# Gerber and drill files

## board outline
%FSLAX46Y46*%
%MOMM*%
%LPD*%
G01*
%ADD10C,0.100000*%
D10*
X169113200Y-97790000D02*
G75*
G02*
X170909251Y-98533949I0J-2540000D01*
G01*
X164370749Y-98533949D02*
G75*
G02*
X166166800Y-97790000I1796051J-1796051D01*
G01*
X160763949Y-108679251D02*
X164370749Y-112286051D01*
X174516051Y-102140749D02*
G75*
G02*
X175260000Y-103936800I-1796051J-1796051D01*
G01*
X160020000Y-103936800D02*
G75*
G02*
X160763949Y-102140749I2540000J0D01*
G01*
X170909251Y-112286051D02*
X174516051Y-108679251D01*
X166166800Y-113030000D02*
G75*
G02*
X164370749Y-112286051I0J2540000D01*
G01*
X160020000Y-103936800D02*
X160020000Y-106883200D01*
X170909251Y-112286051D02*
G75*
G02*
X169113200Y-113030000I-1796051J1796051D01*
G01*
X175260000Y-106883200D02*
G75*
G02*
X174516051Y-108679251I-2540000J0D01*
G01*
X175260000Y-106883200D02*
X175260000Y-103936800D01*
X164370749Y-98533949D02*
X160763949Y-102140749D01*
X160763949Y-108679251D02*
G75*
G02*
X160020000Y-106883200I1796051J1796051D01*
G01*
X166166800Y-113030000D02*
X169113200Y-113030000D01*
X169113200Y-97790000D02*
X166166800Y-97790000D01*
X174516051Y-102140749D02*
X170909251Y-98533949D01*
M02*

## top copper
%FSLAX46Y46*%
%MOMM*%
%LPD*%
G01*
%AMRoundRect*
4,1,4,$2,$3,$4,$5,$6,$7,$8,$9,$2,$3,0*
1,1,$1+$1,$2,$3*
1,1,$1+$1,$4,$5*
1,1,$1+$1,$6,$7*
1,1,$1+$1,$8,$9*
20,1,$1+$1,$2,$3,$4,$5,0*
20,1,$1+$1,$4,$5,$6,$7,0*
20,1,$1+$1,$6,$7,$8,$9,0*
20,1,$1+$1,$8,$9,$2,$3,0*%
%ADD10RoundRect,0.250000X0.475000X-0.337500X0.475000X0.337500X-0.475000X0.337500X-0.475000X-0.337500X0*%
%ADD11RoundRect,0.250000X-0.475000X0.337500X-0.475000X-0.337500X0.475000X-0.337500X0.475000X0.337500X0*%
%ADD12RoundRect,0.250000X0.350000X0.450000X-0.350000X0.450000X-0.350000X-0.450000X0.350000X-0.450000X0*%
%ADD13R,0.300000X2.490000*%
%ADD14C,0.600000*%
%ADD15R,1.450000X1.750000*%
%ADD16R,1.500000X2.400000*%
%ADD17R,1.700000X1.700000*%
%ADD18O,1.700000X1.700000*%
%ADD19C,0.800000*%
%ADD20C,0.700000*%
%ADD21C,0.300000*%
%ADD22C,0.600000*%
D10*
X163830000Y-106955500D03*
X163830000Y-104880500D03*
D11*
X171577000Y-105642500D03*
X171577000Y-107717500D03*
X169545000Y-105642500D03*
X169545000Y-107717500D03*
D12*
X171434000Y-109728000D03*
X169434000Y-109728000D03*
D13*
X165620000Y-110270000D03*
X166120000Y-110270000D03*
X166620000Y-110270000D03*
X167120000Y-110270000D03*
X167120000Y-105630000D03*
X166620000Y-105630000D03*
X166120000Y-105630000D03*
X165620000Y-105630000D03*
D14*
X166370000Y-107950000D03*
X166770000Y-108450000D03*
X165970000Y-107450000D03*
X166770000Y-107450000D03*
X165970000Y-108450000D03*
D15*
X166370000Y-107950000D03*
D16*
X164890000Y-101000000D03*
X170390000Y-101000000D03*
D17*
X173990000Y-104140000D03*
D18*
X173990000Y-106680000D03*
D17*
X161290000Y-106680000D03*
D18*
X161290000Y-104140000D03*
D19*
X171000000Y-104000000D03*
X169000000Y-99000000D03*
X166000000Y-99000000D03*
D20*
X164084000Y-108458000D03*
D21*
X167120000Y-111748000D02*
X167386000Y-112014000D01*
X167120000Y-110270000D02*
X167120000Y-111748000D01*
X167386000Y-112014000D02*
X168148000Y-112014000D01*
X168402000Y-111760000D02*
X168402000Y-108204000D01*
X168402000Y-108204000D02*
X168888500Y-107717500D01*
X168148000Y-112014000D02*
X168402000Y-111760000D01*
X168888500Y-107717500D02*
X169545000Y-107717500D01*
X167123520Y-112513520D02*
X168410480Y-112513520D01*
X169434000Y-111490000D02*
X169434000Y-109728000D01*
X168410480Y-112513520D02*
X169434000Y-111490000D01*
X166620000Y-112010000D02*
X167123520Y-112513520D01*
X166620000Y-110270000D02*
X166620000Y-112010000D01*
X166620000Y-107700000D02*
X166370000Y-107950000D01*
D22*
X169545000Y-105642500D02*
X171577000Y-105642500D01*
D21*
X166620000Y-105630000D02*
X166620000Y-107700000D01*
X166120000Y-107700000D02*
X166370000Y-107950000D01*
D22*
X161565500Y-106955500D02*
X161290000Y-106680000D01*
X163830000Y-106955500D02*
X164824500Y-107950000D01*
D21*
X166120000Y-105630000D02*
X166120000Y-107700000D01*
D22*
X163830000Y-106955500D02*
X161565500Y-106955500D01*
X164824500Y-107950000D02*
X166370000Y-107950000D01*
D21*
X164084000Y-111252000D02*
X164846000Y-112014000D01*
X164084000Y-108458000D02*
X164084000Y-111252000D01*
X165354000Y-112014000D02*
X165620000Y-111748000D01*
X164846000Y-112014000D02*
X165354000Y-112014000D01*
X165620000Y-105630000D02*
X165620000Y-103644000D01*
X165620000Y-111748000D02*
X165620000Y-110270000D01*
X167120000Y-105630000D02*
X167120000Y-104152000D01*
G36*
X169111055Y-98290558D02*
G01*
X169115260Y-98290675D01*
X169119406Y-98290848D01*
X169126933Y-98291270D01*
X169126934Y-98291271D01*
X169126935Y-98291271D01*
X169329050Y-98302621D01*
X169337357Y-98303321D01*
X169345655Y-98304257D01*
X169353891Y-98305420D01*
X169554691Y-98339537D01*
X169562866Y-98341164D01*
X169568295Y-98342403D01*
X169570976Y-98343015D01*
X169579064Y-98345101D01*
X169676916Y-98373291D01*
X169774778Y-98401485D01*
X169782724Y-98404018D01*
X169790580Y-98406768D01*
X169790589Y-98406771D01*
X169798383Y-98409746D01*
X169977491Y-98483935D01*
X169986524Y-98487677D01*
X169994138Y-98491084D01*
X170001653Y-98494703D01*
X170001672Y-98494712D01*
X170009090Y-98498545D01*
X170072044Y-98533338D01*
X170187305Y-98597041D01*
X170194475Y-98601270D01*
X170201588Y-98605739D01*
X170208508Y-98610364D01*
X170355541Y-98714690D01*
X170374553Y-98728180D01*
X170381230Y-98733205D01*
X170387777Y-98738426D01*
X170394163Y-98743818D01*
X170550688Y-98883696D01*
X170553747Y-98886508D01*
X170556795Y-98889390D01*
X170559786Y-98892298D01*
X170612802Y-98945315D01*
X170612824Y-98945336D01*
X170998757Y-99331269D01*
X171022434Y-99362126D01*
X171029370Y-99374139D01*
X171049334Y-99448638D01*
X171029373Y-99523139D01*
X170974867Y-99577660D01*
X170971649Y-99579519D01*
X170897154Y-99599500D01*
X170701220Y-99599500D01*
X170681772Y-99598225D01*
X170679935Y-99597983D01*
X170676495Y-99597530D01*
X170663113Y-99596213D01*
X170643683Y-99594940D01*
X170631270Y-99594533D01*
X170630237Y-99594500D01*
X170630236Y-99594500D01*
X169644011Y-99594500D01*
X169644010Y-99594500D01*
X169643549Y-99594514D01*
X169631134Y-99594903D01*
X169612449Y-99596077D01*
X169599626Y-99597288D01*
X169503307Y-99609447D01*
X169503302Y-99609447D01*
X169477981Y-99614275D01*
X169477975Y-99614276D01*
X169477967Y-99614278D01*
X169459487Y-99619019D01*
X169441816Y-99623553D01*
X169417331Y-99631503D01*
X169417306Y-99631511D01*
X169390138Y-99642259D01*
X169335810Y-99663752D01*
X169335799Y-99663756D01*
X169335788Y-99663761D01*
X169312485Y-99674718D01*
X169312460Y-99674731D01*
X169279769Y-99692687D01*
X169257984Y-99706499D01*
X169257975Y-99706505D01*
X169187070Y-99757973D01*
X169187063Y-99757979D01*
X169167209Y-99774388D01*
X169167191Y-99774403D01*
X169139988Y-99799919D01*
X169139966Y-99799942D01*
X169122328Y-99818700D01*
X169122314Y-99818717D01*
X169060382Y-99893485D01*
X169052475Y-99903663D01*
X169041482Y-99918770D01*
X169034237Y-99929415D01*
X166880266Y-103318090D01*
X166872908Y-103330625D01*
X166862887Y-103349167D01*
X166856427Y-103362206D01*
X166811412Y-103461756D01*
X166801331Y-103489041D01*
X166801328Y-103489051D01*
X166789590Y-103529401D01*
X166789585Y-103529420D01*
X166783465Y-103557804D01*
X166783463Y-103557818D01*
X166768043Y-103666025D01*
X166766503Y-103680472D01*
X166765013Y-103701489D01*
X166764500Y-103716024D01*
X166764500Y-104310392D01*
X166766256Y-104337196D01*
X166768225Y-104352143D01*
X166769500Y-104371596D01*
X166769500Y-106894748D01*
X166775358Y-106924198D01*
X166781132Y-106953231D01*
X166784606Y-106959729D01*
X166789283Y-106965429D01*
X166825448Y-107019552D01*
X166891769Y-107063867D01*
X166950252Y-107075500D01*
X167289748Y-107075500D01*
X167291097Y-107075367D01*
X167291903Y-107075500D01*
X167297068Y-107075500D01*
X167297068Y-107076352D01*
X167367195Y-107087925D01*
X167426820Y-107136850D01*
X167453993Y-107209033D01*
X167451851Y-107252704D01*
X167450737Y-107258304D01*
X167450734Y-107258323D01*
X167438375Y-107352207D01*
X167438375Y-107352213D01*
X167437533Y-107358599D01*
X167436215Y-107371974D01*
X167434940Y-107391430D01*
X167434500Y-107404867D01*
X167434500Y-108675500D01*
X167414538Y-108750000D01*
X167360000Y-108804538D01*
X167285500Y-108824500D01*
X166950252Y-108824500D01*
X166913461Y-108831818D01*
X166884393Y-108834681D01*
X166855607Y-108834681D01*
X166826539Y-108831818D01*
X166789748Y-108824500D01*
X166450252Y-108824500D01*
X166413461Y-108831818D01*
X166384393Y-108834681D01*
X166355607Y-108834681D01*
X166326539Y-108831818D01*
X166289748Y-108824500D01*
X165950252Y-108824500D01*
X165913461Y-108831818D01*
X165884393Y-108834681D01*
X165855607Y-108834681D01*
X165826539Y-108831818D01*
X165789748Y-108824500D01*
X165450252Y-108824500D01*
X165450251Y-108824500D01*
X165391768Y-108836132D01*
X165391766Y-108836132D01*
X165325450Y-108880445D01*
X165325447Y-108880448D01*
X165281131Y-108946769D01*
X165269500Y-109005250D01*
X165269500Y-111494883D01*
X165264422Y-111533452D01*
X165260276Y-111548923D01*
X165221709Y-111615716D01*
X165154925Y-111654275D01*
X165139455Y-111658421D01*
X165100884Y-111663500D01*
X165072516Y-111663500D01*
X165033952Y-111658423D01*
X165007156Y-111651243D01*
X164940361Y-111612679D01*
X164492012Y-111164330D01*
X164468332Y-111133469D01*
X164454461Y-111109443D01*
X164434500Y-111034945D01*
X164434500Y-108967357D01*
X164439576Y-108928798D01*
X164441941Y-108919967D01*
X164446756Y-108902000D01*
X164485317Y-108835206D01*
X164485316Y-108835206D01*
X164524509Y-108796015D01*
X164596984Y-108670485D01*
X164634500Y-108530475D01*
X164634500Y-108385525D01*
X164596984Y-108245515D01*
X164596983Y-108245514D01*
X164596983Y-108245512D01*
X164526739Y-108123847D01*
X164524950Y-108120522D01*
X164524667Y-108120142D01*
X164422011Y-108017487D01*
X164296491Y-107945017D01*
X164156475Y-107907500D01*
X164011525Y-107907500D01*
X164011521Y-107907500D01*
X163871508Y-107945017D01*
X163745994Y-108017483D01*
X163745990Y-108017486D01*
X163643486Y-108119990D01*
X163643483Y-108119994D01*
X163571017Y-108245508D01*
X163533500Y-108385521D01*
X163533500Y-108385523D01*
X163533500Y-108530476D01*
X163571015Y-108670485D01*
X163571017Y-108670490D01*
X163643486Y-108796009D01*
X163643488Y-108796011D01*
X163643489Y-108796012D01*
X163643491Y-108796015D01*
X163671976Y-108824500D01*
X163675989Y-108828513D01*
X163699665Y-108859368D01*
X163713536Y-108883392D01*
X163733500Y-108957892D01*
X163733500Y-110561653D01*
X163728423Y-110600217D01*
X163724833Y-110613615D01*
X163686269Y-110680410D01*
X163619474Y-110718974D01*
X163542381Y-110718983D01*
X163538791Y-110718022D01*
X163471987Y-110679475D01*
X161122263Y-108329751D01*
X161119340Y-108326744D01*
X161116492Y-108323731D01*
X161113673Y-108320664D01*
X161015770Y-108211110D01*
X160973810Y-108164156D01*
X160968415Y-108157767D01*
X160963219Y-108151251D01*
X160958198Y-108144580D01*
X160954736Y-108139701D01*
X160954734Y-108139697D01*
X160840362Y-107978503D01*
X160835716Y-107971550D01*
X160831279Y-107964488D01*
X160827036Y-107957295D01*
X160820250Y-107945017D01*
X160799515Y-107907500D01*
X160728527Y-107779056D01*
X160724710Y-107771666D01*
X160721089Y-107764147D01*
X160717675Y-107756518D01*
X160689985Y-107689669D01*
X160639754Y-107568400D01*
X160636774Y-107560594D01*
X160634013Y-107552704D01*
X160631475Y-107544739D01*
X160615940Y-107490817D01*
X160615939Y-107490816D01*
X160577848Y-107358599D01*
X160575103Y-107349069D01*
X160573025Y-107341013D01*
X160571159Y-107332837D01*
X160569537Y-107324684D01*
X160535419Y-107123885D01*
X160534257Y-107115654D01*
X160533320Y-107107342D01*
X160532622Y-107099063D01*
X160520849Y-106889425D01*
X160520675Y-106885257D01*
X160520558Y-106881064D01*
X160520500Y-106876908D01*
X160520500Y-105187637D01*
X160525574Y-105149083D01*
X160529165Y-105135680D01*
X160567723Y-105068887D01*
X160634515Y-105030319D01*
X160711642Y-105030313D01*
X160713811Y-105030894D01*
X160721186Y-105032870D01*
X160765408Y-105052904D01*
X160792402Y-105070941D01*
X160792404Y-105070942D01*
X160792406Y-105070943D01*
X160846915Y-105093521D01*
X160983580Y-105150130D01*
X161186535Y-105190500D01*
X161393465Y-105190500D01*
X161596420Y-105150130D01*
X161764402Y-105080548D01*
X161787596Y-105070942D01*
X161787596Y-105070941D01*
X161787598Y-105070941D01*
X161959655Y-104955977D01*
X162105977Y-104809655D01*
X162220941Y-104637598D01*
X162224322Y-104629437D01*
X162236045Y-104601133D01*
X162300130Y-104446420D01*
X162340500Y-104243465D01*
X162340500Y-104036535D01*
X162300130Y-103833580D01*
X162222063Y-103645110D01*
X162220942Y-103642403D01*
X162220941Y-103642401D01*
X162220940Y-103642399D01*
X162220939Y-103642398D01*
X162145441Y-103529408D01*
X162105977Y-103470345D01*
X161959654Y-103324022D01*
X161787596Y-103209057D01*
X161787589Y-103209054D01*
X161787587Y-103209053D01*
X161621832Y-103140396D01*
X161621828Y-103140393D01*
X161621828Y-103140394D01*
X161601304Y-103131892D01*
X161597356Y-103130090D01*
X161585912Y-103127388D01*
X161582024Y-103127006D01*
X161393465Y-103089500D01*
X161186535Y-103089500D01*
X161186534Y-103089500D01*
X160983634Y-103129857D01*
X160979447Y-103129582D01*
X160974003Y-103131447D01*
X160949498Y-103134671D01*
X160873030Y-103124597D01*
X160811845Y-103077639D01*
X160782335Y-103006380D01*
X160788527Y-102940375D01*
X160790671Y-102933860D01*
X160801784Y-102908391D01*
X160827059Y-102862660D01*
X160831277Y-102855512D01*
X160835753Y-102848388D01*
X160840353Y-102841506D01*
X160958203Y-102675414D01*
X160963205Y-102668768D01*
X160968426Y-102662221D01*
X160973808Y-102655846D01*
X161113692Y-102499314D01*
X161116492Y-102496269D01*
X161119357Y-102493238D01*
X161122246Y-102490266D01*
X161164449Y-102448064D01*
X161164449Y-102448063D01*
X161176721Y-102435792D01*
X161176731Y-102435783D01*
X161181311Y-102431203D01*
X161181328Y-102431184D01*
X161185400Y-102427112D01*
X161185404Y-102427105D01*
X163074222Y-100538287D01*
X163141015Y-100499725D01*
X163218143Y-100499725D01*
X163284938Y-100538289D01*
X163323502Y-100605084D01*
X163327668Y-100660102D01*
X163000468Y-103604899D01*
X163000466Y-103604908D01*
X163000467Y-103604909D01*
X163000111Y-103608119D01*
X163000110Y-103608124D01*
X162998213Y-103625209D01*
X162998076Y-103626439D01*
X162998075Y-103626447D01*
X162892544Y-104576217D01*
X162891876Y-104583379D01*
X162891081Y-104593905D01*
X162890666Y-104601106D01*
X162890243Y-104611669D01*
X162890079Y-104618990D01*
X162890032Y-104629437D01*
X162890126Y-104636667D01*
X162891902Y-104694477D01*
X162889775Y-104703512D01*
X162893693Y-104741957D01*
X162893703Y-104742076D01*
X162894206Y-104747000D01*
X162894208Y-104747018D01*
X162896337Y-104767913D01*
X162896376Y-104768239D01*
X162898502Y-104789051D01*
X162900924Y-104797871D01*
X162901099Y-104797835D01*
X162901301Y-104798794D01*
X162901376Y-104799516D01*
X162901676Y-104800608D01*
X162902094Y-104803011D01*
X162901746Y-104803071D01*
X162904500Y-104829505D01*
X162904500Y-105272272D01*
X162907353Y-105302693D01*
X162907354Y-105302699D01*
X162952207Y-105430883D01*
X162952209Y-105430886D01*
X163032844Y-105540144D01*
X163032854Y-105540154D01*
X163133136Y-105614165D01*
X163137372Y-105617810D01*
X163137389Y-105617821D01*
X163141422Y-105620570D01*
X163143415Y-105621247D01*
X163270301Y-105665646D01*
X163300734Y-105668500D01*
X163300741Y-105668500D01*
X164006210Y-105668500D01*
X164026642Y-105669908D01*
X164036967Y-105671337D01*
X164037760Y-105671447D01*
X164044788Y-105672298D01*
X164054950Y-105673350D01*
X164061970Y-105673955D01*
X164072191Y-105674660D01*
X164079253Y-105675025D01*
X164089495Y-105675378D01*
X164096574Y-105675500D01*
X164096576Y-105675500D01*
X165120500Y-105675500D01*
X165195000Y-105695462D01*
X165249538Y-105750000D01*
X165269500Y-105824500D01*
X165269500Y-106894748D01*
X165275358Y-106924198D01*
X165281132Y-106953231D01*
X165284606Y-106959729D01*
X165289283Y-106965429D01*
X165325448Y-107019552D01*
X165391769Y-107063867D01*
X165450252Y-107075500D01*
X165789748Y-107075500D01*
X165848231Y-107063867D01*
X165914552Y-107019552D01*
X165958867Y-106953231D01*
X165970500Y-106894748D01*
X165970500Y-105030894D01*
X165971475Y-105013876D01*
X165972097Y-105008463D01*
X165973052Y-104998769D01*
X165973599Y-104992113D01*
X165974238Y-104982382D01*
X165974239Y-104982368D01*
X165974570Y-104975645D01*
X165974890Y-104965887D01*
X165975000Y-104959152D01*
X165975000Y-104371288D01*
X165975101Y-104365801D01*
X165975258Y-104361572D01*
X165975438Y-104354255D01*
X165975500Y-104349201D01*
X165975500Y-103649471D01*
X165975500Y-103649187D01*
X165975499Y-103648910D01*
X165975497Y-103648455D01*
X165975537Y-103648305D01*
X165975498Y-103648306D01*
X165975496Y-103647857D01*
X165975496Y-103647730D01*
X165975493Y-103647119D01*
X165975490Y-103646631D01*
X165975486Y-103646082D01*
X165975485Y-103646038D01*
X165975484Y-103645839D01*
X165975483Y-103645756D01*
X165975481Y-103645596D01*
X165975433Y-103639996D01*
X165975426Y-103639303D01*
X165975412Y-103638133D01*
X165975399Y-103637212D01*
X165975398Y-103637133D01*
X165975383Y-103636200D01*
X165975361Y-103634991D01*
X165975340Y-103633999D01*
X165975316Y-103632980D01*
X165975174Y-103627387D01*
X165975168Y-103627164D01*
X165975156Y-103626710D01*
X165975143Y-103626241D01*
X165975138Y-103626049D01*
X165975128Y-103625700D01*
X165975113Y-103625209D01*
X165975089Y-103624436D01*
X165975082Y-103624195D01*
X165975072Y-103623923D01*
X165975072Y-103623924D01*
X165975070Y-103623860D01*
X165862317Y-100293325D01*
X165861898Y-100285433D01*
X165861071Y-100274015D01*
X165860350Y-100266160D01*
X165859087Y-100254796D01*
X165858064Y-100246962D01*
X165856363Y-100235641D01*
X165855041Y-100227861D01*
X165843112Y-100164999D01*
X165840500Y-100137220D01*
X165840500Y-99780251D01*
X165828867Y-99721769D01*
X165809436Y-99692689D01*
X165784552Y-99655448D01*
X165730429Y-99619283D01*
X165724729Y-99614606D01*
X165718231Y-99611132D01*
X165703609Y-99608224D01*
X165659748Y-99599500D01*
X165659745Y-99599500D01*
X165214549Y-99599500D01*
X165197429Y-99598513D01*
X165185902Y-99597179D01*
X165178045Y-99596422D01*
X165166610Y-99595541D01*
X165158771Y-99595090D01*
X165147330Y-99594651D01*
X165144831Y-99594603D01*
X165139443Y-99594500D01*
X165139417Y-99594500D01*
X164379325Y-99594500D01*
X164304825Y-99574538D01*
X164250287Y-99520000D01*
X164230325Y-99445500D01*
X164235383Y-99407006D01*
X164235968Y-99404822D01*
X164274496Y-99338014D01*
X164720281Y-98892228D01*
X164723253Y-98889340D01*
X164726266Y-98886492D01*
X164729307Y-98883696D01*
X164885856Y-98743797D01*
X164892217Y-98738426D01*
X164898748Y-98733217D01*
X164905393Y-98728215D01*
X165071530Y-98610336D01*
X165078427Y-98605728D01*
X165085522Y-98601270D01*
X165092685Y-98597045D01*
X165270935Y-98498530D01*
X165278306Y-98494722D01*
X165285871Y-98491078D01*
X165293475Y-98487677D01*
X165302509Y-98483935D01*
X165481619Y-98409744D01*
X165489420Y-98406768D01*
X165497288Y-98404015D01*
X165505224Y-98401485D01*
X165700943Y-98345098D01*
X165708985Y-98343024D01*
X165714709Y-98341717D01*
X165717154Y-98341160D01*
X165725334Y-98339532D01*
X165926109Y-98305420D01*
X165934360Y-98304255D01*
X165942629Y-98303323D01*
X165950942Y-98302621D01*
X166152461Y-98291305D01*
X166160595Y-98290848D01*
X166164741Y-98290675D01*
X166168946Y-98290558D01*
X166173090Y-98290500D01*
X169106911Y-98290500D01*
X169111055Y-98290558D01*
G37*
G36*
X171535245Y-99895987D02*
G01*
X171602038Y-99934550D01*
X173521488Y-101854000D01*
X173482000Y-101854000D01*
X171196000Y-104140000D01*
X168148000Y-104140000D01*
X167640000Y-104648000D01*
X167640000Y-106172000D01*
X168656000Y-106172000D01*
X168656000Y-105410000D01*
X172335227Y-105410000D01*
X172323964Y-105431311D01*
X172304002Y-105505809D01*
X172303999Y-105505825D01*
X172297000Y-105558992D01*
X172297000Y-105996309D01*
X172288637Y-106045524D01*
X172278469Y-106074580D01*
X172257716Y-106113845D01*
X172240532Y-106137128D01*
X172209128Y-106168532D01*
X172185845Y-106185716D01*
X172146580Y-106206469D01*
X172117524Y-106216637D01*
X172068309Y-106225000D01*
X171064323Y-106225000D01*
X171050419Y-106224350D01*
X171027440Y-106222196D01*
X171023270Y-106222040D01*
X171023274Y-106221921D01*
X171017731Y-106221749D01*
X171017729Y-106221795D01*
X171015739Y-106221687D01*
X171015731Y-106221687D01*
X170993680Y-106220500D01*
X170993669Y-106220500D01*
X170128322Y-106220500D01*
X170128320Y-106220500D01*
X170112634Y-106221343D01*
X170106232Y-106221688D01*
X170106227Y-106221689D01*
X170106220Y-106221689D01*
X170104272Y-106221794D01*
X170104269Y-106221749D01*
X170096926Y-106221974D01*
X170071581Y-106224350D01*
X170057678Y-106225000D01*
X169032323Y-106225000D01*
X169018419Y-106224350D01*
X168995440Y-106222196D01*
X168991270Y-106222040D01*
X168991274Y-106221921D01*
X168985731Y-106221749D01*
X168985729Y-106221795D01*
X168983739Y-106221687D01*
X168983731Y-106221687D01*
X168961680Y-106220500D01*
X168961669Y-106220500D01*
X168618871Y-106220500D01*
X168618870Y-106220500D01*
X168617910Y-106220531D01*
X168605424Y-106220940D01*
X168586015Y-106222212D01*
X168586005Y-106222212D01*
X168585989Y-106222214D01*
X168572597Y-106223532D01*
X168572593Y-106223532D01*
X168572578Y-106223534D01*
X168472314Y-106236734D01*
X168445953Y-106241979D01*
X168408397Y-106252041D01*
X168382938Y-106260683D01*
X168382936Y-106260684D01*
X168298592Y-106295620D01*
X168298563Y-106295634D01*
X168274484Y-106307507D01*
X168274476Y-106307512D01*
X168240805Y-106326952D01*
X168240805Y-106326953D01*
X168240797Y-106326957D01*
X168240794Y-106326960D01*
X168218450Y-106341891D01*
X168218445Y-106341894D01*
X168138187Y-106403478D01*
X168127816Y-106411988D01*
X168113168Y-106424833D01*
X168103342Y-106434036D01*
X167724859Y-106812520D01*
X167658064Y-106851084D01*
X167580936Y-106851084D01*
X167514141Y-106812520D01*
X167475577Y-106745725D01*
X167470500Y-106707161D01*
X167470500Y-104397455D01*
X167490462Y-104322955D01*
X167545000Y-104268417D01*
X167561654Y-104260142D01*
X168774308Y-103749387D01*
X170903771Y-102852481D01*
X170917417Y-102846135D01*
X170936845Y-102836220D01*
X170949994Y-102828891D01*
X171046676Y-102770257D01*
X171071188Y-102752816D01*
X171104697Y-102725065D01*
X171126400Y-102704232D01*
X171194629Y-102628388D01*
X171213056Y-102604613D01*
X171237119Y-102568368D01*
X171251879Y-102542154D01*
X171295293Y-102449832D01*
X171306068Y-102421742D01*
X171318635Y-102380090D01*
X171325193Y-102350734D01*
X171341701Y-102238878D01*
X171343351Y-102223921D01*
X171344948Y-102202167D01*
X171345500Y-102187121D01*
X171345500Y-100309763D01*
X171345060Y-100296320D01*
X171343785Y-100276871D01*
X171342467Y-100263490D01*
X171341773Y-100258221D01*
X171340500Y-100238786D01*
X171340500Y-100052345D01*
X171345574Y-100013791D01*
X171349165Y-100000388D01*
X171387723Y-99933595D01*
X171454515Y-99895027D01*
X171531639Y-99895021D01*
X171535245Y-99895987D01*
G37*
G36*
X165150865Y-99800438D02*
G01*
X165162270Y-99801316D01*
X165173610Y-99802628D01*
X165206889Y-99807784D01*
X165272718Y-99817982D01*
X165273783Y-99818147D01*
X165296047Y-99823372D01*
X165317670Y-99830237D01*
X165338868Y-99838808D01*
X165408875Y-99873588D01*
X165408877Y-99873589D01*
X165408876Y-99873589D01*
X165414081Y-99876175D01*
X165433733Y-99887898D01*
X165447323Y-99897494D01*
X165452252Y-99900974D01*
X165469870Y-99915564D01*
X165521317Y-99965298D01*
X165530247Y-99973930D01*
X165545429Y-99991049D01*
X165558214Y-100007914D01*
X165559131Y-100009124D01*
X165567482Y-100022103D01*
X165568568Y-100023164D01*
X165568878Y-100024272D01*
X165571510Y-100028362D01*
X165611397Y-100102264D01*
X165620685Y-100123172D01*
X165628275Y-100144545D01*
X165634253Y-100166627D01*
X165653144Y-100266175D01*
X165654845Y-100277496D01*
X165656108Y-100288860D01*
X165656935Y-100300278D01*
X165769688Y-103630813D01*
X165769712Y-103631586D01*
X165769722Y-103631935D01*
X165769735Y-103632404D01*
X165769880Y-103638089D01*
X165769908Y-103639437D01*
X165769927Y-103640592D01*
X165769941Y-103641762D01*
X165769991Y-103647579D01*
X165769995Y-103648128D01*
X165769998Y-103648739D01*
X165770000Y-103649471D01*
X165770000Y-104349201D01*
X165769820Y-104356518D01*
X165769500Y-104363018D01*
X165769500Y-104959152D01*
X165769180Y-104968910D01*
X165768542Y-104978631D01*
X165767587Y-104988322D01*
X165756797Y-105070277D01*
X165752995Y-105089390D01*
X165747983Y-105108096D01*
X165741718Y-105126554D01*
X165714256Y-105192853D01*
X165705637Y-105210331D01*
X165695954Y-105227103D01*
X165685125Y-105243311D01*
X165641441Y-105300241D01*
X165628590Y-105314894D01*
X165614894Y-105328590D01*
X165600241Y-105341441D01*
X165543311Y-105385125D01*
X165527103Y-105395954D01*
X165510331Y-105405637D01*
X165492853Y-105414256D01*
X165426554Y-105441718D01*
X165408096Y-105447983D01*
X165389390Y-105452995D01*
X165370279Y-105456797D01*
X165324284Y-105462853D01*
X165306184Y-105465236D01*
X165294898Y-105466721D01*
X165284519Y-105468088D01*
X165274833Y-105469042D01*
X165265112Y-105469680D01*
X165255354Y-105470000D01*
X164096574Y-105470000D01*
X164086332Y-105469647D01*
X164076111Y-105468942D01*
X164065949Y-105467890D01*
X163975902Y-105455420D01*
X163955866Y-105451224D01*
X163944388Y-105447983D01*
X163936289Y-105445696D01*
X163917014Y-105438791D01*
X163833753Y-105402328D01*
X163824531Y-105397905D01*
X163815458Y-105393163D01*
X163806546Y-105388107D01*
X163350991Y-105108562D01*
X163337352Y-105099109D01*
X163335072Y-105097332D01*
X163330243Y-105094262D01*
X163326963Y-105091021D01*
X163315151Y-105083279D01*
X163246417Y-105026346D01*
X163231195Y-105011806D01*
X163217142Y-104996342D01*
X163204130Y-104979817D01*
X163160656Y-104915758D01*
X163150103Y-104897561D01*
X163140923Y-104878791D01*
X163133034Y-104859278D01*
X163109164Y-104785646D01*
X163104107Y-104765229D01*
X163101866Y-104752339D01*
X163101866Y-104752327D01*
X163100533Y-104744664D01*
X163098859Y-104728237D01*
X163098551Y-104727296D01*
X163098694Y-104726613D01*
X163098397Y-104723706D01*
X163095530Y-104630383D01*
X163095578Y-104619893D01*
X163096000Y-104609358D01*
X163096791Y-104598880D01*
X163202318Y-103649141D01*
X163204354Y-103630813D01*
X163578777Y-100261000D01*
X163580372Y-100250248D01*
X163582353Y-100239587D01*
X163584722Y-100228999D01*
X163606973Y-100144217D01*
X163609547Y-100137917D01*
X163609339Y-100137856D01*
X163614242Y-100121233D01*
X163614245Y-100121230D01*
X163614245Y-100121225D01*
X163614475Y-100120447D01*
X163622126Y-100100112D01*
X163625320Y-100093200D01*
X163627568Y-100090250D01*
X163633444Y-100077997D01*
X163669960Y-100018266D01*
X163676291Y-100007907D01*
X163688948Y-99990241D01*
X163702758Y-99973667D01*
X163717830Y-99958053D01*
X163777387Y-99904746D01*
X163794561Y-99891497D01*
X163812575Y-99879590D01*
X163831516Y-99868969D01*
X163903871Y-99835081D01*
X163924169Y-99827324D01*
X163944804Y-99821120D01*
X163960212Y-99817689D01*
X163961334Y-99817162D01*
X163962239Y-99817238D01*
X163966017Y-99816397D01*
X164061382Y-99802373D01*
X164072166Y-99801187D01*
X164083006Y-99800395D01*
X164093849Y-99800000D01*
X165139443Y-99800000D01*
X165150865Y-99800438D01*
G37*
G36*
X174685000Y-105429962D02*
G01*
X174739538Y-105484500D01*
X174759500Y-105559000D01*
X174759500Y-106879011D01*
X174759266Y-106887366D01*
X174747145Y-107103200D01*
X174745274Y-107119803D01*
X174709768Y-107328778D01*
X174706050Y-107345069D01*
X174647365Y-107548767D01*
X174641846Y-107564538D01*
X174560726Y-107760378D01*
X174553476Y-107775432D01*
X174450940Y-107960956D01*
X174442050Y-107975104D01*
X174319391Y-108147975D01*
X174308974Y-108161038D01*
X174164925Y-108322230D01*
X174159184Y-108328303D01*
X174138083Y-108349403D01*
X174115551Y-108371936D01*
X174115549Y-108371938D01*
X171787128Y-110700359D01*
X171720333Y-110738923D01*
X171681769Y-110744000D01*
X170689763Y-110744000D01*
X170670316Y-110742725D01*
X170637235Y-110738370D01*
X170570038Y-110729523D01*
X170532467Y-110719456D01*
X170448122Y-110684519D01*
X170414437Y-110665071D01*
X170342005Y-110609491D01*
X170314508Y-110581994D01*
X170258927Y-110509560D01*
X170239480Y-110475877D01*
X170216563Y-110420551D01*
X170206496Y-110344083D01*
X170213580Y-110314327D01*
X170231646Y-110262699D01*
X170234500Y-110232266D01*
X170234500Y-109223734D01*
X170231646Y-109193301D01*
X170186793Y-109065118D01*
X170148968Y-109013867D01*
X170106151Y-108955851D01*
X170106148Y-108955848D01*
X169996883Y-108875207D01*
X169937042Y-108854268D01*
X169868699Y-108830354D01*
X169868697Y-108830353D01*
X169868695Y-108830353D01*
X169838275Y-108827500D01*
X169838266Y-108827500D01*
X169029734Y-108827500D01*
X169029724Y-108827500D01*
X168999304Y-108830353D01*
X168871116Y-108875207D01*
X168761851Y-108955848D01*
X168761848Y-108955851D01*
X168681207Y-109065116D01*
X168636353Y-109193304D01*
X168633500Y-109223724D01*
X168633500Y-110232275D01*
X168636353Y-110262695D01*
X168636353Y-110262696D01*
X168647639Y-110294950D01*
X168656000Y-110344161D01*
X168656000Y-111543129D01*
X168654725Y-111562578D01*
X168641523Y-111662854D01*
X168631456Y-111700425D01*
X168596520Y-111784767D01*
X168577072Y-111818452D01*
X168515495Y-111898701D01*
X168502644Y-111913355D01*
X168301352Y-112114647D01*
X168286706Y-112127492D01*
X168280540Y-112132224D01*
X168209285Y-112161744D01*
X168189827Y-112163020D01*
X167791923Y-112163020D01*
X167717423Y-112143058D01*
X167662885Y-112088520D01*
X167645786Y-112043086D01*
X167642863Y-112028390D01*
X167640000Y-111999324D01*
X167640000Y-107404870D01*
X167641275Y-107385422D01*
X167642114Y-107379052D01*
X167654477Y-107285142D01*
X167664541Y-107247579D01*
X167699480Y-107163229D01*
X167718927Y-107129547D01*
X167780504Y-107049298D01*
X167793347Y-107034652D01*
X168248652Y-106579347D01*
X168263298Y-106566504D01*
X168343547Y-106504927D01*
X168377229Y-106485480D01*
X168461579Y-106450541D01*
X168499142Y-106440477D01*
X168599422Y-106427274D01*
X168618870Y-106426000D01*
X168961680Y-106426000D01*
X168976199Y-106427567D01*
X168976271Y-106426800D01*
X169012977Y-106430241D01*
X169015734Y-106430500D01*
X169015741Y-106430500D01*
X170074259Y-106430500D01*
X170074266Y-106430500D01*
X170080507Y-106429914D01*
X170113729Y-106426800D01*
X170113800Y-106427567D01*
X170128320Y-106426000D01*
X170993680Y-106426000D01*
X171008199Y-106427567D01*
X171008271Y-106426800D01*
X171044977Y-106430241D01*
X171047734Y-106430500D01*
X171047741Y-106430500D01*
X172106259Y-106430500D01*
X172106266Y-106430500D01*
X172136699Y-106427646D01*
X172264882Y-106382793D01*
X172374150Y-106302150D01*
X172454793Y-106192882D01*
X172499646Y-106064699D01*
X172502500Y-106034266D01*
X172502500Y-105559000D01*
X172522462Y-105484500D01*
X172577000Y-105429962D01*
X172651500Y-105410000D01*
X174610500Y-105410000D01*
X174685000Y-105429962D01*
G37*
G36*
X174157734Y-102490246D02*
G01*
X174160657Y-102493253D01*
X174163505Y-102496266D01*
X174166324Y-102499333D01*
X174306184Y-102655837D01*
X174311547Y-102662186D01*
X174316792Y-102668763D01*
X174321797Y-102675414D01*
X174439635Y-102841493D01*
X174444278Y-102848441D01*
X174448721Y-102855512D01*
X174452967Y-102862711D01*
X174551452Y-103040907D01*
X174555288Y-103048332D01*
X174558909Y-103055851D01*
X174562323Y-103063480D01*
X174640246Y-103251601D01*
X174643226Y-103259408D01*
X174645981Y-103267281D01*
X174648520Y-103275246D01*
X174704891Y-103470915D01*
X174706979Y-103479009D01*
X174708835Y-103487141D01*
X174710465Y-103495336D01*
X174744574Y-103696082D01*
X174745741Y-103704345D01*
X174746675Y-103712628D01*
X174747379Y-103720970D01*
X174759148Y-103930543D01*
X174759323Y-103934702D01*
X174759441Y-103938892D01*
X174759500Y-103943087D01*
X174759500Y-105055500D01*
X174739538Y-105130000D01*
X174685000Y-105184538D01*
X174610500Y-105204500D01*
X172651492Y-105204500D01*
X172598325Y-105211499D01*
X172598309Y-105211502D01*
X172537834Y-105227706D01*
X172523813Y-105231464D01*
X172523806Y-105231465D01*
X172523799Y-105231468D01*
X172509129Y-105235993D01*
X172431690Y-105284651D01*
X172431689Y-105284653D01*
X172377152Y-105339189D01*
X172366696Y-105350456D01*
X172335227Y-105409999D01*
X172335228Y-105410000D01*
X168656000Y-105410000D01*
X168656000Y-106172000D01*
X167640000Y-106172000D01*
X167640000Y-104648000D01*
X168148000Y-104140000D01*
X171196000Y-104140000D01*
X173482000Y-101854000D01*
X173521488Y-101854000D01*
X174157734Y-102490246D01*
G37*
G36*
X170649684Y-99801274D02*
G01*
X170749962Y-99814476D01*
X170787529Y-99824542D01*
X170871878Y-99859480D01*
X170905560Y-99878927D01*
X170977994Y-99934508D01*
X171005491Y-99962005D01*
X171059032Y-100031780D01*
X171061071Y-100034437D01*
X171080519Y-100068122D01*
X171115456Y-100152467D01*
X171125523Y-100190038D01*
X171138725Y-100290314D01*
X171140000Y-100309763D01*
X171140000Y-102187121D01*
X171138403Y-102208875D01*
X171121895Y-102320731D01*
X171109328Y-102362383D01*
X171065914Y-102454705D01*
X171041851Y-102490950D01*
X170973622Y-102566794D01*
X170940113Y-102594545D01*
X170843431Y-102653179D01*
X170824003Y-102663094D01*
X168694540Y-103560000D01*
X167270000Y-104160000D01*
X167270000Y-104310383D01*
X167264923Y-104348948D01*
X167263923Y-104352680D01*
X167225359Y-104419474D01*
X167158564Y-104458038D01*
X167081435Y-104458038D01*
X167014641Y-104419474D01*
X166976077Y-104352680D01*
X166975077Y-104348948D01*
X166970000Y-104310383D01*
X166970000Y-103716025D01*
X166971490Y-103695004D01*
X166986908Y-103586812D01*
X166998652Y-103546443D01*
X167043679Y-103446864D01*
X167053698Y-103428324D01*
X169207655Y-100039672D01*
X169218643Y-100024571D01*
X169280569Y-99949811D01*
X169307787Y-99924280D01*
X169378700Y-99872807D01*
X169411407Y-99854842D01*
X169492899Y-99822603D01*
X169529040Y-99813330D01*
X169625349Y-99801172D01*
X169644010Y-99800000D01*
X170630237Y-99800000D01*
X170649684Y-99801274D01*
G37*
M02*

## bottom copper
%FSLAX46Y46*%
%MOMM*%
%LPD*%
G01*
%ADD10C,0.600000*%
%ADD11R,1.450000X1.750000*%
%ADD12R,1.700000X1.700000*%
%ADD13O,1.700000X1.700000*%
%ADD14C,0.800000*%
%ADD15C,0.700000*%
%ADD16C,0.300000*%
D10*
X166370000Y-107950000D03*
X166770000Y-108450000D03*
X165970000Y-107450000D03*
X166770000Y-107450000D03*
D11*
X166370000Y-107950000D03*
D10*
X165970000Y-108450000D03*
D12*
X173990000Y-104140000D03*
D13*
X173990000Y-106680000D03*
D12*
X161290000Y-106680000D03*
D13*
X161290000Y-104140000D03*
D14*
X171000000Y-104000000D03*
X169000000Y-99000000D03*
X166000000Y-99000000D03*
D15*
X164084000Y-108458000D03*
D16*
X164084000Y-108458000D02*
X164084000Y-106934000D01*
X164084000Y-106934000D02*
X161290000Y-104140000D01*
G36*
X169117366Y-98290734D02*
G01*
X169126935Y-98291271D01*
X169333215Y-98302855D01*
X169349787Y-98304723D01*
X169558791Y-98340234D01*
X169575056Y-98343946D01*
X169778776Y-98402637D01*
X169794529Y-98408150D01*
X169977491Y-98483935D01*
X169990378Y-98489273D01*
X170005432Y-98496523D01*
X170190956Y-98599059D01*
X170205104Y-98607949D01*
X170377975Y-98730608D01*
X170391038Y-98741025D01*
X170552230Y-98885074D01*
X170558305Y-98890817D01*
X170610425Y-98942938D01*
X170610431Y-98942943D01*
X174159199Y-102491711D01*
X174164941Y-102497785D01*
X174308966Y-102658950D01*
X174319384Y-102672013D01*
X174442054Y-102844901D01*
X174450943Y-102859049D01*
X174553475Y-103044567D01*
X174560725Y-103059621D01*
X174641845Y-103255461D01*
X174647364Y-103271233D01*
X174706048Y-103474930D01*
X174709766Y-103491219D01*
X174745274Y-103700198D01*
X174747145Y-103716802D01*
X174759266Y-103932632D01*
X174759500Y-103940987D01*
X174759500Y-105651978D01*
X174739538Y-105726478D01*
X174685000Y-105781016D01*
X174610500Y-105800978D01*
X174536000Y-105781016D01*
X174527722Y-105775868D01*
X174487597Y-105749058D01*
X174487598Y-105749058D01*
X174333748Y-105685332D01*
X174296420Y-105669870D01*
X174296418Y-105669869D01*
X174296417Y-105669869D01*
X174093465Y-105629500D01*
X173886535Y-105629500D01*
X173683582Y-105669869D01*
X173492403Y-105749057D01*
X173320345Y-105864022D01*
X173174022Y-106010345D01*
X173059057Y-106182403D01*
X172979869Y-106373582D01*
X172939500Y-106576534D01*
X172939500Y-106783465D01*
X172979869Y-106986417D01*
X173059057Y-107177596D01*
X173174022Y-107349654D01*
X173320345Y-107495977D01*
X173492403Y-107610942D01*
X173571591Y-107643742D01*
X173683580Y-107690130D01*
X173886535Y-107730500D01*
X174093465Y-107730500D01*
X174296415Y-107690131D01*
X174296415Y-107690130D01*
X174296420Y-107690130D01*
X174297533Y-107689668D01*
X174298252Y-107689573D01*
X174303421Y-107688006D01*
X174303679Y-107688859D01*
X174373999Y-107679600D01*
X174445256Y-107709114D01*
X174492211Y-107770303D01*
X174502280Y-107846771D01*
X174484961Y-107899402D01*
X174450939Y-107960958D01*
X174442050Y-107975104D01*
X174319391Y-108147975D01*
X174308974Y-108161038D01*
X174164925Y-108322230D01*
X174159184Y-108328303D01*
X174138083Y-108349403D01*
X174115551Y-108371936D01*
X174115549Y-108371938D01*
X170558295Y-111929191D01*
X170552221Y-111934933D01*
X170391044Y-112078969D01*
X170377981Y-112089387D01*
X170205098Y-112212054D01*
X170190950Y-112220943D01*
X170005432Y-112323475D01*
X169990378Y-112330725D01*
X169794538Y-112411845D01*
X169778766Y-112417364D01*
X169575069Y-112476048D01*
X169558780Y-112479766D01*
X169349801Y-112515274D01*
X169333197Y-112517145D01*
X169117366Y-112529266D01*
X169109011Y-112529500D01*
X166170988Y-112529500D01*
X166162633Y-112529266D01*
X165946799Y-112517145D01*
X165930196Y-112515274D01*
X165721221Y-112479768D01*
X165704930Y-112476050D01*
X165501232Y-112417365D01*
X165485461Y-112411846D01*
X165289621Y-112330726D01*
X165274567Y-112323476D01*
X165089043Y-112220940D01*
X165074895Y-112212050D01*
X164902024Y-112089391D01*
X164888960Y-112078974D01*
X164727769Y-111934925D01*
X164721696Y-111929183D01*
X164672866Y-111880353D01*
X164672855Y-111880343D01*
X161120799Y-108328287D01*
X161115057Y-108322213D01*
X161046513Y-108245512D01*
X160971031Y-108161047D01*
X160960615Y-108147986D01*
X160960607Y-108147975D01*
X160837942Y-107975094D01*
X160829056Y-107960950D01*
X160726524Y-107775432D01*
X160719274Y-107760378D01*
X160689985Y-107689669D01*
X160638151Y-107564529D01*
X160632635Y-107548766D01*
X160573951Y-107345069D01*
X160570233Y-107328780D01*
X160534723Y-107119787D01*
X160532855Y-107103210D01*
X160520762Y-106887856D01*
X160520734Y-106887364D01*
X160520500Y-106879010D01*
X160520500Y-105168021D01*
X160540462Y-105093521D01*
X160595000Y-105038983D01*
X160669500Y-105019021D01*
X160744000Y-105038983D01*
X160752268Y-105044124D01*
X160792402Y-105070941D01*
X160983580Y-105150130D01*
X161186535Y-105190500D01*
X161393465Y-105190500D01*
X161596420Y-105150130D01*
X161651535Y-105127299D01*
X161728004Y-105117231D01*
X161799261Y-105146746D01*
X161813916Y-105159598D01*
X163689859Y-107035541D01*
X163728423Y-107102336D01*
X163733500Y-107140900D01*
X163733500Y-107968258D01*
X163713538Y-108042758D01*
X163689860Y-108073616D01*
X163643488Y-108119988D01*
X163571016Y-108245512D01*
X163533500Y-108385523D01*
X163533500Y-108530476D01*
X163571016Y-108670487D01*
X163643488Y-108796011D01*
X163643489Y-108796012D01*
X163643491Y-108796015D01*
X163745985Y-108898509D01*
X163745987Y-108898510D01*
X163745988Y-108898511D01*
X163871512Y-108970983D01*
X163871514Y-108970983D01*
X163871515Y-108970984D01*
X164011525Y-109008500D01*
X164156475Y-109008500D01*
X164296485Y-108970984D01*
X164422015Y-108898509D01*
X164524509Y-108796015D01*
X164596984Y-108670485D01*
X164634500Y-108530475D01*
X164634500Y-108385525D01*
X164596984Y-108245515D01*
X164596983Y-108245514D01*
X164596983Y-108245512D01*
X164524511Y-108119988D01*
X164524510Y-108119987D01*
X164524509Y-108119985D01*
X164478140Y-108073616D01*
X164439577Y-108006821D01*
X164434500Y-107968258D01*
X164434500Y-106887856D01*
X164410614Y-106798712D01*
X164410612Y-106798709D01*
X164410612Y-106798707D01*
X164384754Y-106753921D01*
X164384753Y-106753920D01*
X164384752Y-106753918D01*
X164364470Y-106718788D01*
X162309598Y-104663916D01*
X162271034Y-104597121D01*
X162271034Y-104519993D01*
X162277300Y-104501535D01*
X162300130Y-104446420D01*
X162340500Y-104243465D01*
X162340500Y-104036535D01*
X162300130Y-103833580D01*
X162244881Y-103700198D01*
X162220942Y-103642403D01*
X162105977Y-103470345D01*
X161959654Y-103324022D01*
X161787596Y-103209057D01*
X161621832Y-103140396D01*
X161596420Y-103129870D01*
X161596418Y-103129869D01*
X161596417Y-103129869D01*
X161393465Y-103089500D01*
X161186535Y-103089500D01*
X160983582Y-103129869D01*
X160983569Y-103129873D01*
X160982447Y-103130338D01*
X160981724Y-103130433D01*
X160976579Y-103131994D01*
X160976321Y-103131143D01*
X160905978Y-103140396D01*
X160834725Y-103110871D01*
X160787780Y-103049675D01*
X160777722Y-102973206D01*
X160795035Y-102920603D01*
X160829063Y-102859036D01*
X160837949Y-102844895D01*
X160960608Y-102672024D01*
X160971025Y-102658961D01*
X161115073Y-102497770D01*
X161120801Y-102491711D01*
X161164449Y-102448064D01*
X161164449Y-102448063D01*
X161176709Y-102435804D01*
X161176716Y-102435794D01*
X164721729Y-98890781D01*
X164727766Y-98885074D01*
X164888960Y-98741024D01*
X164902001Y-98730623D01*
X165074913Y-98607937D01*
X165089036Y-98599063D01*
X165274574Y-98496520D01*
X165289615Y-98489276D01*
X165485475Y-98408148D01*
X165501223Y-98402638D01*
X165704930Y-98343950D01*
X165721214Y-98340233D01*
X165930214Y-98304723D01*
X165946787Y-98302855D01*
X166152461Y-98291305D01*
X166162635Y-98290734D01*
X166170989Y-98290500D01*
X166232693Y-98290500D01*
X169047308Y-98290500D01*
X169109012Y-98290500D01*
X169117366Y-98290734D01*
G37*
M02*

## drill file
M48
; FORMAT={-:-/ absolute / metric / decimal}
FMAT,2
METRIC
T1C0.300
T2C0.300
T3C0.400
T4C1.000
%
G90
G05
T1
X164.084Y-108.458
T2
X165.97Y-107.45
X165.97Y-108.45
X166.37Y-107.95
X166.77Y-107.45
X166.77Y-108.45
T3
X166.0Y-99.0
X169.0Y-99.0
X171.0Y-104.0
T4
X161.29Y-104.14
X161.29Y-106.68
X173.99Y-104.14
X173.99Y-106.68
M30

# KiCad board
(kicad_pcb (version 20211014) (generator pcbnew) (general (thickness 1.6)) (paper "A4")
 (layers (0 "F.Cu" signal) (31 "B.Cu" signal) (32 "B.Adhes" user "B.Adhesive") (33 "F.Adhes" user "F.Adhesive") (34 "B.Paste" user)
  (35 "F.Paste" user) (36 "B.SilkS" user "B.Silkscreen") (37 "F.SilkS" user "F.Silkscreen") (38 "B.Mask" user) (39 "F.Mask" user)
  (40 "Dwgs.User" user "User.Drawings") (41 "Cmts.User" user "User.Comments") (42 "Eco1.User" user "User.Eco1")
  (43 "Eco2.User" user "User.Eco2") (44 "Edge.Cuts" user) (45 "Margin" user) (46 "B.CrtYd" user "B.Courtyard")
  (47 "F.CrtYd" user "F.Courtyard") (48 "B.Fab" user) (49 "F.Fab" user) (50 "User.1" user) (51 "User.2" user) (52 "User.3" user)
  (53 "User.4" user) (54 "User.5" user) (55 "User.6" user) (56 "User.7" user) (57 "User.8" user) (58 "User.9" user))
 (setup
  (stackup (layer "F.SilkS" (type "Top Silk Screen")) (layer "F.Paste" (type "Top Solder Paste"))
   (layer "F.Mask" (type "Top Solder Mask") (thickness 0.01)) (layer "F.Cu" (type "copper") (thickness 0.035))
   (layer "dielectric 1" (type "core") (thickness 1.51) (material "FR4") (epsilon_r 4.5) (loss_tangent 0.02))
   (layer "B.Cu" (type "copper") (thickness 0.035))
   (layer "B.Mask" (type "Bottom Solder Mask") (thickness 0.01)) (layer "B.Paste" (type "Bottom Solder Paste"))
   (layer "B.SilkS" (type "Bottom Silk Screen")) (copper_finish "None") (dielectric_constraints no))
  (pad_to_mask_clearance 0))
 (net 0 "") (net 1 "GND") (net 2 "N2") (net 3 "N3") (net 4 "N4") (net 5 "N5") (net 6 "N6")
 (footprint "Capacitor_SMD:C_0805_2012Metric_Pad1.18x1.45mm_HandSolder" (layer "F.Cu") (at 163.83 105.918 90)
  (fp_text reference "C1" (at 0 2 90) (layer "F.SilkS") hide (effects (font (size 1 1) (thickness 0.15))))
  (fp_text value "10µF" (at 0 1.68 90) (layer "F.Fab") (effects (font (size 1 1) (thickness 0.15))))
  (pad "1" smd roundrect locked (at -1.0375 0 90) (size 1.175 1.45) (layers "F.Cu" "F.Paste" "F.Mask") (roundrect_rratio 0.212766)
   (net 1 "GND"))
  (pad "2" smd roundrect locked (at 1.0375 0 90) (size 1.175 1.45) (layers "F.Cu" "F.Paste" "F.Mask") (roundrect_rratio 0.212766)
   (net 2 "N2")))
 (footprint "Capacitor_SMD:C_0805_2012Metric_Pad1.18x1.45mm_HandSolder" (layer "F.Cu") (at 171.577 106.68 -90)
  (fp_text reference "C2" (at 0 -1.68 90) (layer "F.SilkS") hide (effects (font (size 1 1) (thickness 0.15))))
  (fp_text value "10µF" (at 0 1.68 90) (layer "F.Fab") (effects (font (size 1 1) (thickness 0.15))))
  (pad "1" smd roundrect locked (at -1.0375 0 270) (size 1.175 1.45) (layers "F.Cu" "F.Paste" "F.Mask") (roundrect_rratio 0.212766)
   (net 1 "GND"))
  (pad "2" smd roundrect locked (at 1.0375 0 270) (size 1.175 1.45) (layers "F.Cu" "F.Paste" "F.Mask") (roundrect_rratio 0.212766)
   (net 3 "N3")))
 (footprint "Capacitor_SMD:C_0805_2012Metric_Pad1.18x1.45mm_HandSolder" (layer "F.Cu") (at 169.545 106.68 -90)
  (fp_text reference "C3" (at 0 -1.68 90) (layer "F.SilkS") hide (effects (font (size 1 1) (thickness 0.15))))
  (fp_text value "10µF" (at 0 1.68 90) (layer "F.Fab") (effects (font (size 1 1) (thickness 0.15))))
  (pad "1" smd roundrect locked (at -1.0375 0 270) (size 1.175 1.45) (layers "F.Cu" "F.Paste" "F.Mask") (roundrect_rratio 0.212766)
   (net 1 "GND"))
  (pad "2" smd roundrect locked (at 1.0375 0 270) (size 1.175 1.45) (layers "F.Cu" "F.Paste" "F.Mask") (roundrect_rratio 0.212766)
   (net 3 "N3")))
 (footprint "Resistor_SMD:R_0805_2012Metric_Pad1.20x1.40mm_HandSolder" (layer "F.Cu") (at 170.434 109.728 180)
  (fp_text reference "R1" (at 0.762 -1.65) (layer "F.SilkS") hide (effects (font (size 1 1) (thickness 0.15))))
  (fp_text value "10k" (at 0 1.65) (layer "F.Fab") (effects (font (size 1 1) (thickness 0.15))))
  (pad "1" smd roundrect locked (at -1 0 180) (size 1.2 1.4) (layers "F.Cu" "F.Paste" "F.Mask") (roundrect_rratio 0.208333) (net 3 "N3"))
  (pad "2" smd roundrect locked (at 1 0 180) (size 1.2 1.4) (layers "F.Cu" "F.Paste" "F.Mask") (roundrect_rratio 0.208333) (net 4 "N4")))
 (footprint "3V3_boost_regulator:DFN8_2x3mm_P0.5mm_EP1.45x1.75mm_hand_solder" (layer "F.Cu") (at 166.37 107.95 90)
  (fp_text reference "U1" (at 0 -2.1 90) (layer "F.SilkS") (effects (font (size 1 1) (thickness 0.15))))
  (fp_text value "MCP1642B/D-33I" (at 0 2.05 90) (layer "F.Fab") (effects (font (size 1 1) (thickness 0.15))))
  (pad "" smd roundrect (at -0.5 0 90) (size 0.55 1.3) (layers "F.Paste") (roundrect_rratio 0.25))
  (pad "" smd roundrect (at 0.5 0 90) (size 0.55 1.3) (layers "F.Paste") (roundrect_rratio 0.25))
  (pad "" smd roundrect (at 0 0.45 90) (size 1.6 0.456) (layers "F.Paste") (roundrect_rratio 0.25))
  (pad "" smd roundrect (at 0 -0.45 90) (size 1.6 0.456) (layers "F.Paste") (roundrect_rratio 0.25))
  (pad "1" smd rect (at -2.32 -0.75 90) (size 2.49 0.3) (layers "F.Cu" "F.Paste" "F.Mask") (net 2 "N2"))
  (pad "2" smd rect (at -2.32 -0.25 90) (size 2.49 0.3) (layers "F.Cu" "F.Paste" "F.Mask") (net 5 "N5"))
  (pad "3" smd rect (at -2.32 0.25 90) (size 2.49 0.3) (layers "F.Cu" "F.Paste" "F.Mask") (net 4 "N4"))
  (pad "4" smd rect (at -2.32 0.75 90) (size 2.49 0.3) (layers "F.Cu" "F.Paste" "F.Mask") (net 3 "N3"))
  (pad "5" smd rect (at 2.32 0.75 90) (size 2.49 0.3) (layers "F.Cu" "F.Paste" "F.Mask") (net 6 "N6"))
  (pad "6" smd rect (at 2.32 0.25 90) (size 2.49 0.3) (layers "F.Cu" "F.Paste" "F.Mask") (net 1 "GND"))
  (pad "7" smd rect (at 2.32 -0.25 90) (size 2.49 0.3) (layers "F.Cu" "F.Paste" "F.Mask") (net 1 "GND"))
  (pad "8" smd rect (at 2.32 -0.75 90) (size 2.49 0.3) (layers "F.Cu" "F.Paste" "F.Mask") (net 2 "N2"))
  (pad "9" thru_hole circle (at 0 0 90) (size 0.6 0.6) (drill 0.3) (layers *.Cu *.Mask) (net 1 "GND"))
  (pad "9" thru_hole circle (at -0.5 0.4 90) (size 0.6 0.6) (drill 0.3) (layers *.Cu *.Mask) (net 1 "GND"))
  (pad "9" thru_hole circle (at 0.5 -0.4 90) (size 0.6 0.6) (drill 0.3) (layers *.Cu *.Mask) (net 1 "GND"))
  (pad "9" thru_hole circle (at 0.5 0.4 90) (size 0.6 0.6) (drill 0.3) (layers *.Cu *.Mask) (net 1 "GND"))
  (pad "9" smd rect (at 0 0 90) (size 1.75 1.45) (layers "B.Cu" "B.Mask") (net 1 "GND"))
  (pad "9" thru_hole circle (at -0.5 -0.4 90) (size 0.6 0.6) (drill 0.3) (layers *.Cu *.Mask) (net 1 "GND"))
  (pad "9" smd rect (at 0 0 90) (size 1.75 1.45) (layers "F.Cu" "F.Mask") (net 1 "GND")))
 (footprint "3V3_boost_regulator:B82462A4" (layer "F.Cu") (at 167.64 101)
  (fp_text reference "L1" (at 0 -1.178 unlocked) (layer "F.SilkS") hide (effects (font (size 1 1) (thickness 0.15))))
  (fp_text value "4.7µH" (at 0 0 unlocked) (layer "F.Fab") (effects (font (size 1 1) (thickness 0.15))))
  (pad "1" smd rect (at -2.75 0) (size 1.5 2.4) (layers "F.Cu" "F.Paste" "F.Mask") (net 2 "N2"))
  (pad "2" smd rect (at 2.75 0) (size 1.5 2.4) (layers "F.Cu" "F.Paste" "F.Mask") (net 6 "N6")))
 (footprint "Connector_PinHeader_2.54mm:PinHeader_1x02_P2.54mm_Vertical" (layer "B.Cu") (at 173.99 104.14 180)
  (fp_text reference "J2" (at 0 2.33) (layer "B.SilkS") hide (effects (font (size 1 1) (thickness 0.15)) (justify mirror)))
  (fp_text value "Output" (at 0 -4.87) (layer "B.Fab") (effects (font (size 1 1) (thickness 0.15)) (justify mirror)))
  (pad "1" thru_hole rect (at 0 0 180) (size 1.7 1.7) (drill 1) (layers *.Cu *.Mask) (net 1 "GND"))
  (pad "2" thru_hole oval (at 0 -2.54 180) (size 1.7 1.7) (drill 1) (layers *.Cu *.Mask) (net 3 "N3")))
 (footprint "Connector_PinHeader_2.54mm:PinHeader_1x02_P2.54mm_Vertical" (layer "B.Cu") (at 161.29 106.68)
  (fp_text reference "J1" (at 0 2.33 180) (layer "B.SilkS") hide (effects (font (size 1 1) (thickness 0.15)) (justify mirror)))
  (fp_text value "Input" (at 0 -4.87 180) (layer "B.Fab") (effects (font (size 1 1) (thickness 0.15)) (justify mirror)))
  (pad "1" thru_hole rect (at 0 0) (size 1.7 1.7) (drill 1) (layers *.Cu *.Mask) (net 1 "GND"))
  (pad "2" thru_hole oval (at 0 -2.54) (size 1.7 1.7) (drill 1) (layers *.Cu *.Mask) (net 2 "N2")))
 (gr_arc (start 169.1132 97.79) (mid 170.085216 97.983346) (end 170.909251 98.533949) (layer "Edge.Cuts") (width 0.1))
 (gr_arc (start 164.370749 98.533949) (mid 165.194784 97.983347) (end 166.1668 97.79) (layer "Edge.Cuts") (width 0.1))
 (gr_line (start 160.763949 108.679251) (end 164.370749 112.286051) (layer "Edge.Cuts") (width 0.1))
 (gr_arc (start 174.516051 102.140749) (mid 175.066653 102.964784) (end 175.26 103.9368) (layer "Edge.Cuts") (width 0.1))
 (gr_arc (start 160.02 103.9368) (mid 160.213346 102.964784) (end 160.763949 102.140749) (layer "Edge.Cuts") (width 0.1))
 (gr_line (start 170.909251 112.286051) (end 174.516051 108.679251) (layer "Edge.Cuts") (width 0.1))
 (gr_arc (start 166.1668 113.03) (mid 165.194784 112.836654) (end 164.370749 112.286051) (layer "Edge.Cuts") (width 0.1))
 (gr_line (start 160.02 103.9368) (end 160.02 106.8832) (layer "Edge.Cuts") (width 0.1))
 (gr_arc (start 170.909251 112.286051) (mid 170.085216 112.836653) (end 169.1132 113.03) (layer "Edge.Cuts") (width 0.1))
 (gr_arc (start 175.26 106.8832) (mid 175.066654 107.855216) (end 174.516051 108.679251) (layer "Edge.Cuts") (width 0.1))
 (gr_line (start 175.26 106.8832) (end 175.26 103.9368) (layer "Edge.Cuts") (width 0.1))
 (gr_line (start 164.370749 98.533949) (end 160.763949 102.140749) (layer "Edge.Cuts") (width 0.1))
 (gr_arc (start 160.763949 108.679251) (mid 160.213347 107.855216) (end 160.02 106.8832) (layer "Edge.Cuts") (width 0.1))
 (gr_line (start 166.1668 113.03) (end 169.1132 113.03) (layer "Edge.Cuts") (width 0.1))
 (gr_line (start 169.1132 97.79) (end 166.1668 97.79) (layer "Edge.Cuts") (width 0.1))
 (gr_line (start 174.516051 102.140749) (end 170.909251 98.533949) (layer "Edge.Cuts") (width 0.1))
 (segment (start 167.12 111.748) (end 167.386 112.014) (width 0.3) (layer "F.Cu") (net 3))
 (segment (start 167.12 110.27) (end 167.12 111.748) (width 0.3) (layer "F.Cu") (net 3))
 (segment (start 167.386 112.014) (end 168.148 112.014) (width 0.3) (layer "F.Cu") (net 3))
 (segment (start 168.402 111.76) (end 168.402 108.204) (width 0.3) (layer "F.Cu") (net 3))
 (segment (start 168.402 108.204) (end 168.8885 107.7175) (width 0.3) (layer "F.Cu") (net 3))
 (segment (start 168.148 112.014) (end 168.402 111.76) (width 0.3) (layer "F.Cu") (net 3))
 (segment (start 168.8885 107.7175) (end 169.545 107.7175) (width 0.3) (layer "F.Cu") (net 3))
 (segment (start 167.12352 112.51352) (end 168.41048 112.51352) (width 0.3) (layer "F.Cu") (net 4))
 (segment (start 169.434 111.49) (end 169.434 109.728) (width 0.3) (layer "F.Cu") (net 4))
 (segment (start 168.41048 112.51352) (end 169.434 111.49) (width 0.3) (layer "F.Cu") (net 4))
 (segment (start 166.62 112.01) (end 167.12352 112.51352) (width 0.3) (layer "F.Cu") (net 4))
 (segment (start 166.62 110.27) (end 166.62 112.01) (width 0.3) (layer "F.Cu") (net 4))
 (segment (start 166.62 107.7) (end 166.37 107.95) (width 0.3) (layer "F.Cu") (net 1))
 (segment (start 169.545 105.6425) (end 171.577 105.6425) (width 0.6) (layer "F.Cu") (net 1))
 (segment (start 166.62 105.63) (end 166.62 107.7) (width 0.3) (layer "F.Cu") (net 1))
 (segment (start 166.12 107.7) (end 166.37 107.95) (width 0.3) (layer "F.Cu") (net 1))
 (segment (start 161.5655 106.9555) (end 161.29 106.68) (width 0.6) (layer "F.Cu") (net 1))
 (segment (start 163.83 106.9555) (end 164.8245 107.95) (width 0.6) (layer "F.Cu") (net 1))
 (segment (start 166.12 105.63) (end 166.12 107.7) (width 0.3) (layer "F.Cu") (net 1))
 (segment (start 163.83 106.9555) (end 161.5655 106.9555) (width 0.6) (layer "F.Cu") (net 1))
 (segment (start 164.8245 107.95) (end 166.37 107.95) (width 0.6) (layer "F.Cu") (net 1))
 (via (at 171 104) (size 0.8) (drill 0.4) (layers "F.Cu" "B.Cu") (free) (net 1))
 (via (at 169 99) (size 0.8) (drill 0.4) (layers "F.Cu" "B.Cu") (free) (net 1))
 (via (at 166 99) (size 0.8) (drill 0.4) (layers "F.Cu" "B.Cu") (free) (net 1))
 (segment (start 164.084 111.252) (end 164.846 112.014) (width 0.3) (layer "F.Cu") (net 2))
 (segment (start 164.084 108.458) (end 164.084 111.252) (width 0.3) (layer "F.Cu") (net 2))
 (segment (start 165.354 112.014) (end 165.62 111.748) (width 0.3) (layer "F.Cu") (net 2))
 (segment (start 164.846 112.014) (end 165.354 112.014) (width 0.3) (layer "F.Cu") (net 2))
 (segment (start 165.62 105.63) (end 165.62 103.644) (width 0.3) (layer "F.Cu") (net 2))
 (segment (start 165.62 111.748) (end 165.62 110.27) (width 0.3) (layer "F.Cu") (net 2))
 (via (at 164.084 108.458) (size 0.7) (drill 0.3) (layers "F.Cu" "B.Cu") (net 2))
 (segment (start 164.084 108.458) (end 164.084 106.934) (width 0.3) (layer "B.Cu") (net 2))
 (segment (start 164.084 106.934) (end 161.29 104.14) (width 0.3) (layer "B.Cu") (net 2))
 (segment (start 167.12 105.63) (end 167.12 104.152) (width 0.3) (layer "F.Cu") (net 6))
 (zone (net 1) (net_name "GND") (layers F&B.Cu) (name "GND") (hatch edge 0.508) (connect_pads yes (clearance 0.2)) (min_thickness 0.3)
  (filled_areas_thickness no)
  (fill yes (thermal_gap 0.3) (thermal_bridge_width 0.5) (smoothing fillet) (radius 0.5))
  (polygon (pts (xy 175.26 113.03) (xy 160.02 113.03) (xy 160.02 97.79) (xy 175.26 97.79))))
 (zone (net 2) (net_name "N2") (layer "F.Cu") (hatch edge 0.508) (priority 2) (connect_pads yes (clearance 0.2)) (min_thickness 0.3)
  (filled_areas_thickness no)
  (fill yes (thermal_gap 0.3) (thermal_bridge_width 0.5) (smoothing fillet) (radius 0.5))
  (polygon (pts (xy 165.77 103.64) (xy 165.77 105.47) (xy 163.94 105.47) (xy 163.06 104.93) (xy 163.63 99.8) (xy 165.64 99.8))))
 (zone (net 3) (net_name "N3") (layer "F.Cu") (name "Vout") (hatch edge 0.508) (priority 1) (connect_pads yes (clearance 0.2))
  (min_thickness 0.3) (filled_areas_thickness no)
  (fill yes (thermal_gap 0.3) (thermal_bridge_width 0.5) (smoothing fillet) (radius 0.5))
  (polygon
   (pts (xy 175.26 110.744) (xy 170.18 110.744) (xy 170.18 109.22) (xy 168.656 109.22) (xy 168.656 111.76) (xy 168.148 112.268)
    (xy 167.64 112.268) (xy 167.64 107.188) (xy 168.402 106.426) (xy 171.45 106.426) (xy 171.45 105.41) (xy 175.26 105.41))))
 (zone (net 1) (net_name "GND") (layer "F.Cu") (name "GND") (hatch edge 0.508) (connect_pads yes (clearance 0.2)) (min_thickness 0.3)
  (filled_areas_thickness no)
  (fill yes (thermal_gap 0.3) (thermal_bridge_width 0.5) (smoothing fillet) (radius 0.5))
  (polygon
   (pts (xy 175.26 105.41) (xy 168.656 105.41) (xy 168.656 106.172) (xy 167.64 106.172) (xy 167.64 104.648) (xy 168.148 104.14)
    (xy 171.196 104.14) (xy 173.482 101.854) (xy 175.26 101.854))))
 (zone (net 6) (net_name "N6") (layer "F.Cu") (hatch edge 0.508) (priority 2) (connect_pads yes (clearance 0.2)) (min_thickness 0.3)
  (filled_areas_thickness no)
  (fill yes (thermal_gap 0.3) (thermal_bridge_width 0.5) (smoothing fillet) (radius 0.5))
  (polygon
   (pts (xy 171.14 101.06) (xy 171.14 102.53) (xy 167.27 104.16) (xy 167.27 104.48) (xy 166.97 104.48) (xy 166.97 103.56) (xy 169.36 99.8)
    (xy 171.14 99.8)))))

